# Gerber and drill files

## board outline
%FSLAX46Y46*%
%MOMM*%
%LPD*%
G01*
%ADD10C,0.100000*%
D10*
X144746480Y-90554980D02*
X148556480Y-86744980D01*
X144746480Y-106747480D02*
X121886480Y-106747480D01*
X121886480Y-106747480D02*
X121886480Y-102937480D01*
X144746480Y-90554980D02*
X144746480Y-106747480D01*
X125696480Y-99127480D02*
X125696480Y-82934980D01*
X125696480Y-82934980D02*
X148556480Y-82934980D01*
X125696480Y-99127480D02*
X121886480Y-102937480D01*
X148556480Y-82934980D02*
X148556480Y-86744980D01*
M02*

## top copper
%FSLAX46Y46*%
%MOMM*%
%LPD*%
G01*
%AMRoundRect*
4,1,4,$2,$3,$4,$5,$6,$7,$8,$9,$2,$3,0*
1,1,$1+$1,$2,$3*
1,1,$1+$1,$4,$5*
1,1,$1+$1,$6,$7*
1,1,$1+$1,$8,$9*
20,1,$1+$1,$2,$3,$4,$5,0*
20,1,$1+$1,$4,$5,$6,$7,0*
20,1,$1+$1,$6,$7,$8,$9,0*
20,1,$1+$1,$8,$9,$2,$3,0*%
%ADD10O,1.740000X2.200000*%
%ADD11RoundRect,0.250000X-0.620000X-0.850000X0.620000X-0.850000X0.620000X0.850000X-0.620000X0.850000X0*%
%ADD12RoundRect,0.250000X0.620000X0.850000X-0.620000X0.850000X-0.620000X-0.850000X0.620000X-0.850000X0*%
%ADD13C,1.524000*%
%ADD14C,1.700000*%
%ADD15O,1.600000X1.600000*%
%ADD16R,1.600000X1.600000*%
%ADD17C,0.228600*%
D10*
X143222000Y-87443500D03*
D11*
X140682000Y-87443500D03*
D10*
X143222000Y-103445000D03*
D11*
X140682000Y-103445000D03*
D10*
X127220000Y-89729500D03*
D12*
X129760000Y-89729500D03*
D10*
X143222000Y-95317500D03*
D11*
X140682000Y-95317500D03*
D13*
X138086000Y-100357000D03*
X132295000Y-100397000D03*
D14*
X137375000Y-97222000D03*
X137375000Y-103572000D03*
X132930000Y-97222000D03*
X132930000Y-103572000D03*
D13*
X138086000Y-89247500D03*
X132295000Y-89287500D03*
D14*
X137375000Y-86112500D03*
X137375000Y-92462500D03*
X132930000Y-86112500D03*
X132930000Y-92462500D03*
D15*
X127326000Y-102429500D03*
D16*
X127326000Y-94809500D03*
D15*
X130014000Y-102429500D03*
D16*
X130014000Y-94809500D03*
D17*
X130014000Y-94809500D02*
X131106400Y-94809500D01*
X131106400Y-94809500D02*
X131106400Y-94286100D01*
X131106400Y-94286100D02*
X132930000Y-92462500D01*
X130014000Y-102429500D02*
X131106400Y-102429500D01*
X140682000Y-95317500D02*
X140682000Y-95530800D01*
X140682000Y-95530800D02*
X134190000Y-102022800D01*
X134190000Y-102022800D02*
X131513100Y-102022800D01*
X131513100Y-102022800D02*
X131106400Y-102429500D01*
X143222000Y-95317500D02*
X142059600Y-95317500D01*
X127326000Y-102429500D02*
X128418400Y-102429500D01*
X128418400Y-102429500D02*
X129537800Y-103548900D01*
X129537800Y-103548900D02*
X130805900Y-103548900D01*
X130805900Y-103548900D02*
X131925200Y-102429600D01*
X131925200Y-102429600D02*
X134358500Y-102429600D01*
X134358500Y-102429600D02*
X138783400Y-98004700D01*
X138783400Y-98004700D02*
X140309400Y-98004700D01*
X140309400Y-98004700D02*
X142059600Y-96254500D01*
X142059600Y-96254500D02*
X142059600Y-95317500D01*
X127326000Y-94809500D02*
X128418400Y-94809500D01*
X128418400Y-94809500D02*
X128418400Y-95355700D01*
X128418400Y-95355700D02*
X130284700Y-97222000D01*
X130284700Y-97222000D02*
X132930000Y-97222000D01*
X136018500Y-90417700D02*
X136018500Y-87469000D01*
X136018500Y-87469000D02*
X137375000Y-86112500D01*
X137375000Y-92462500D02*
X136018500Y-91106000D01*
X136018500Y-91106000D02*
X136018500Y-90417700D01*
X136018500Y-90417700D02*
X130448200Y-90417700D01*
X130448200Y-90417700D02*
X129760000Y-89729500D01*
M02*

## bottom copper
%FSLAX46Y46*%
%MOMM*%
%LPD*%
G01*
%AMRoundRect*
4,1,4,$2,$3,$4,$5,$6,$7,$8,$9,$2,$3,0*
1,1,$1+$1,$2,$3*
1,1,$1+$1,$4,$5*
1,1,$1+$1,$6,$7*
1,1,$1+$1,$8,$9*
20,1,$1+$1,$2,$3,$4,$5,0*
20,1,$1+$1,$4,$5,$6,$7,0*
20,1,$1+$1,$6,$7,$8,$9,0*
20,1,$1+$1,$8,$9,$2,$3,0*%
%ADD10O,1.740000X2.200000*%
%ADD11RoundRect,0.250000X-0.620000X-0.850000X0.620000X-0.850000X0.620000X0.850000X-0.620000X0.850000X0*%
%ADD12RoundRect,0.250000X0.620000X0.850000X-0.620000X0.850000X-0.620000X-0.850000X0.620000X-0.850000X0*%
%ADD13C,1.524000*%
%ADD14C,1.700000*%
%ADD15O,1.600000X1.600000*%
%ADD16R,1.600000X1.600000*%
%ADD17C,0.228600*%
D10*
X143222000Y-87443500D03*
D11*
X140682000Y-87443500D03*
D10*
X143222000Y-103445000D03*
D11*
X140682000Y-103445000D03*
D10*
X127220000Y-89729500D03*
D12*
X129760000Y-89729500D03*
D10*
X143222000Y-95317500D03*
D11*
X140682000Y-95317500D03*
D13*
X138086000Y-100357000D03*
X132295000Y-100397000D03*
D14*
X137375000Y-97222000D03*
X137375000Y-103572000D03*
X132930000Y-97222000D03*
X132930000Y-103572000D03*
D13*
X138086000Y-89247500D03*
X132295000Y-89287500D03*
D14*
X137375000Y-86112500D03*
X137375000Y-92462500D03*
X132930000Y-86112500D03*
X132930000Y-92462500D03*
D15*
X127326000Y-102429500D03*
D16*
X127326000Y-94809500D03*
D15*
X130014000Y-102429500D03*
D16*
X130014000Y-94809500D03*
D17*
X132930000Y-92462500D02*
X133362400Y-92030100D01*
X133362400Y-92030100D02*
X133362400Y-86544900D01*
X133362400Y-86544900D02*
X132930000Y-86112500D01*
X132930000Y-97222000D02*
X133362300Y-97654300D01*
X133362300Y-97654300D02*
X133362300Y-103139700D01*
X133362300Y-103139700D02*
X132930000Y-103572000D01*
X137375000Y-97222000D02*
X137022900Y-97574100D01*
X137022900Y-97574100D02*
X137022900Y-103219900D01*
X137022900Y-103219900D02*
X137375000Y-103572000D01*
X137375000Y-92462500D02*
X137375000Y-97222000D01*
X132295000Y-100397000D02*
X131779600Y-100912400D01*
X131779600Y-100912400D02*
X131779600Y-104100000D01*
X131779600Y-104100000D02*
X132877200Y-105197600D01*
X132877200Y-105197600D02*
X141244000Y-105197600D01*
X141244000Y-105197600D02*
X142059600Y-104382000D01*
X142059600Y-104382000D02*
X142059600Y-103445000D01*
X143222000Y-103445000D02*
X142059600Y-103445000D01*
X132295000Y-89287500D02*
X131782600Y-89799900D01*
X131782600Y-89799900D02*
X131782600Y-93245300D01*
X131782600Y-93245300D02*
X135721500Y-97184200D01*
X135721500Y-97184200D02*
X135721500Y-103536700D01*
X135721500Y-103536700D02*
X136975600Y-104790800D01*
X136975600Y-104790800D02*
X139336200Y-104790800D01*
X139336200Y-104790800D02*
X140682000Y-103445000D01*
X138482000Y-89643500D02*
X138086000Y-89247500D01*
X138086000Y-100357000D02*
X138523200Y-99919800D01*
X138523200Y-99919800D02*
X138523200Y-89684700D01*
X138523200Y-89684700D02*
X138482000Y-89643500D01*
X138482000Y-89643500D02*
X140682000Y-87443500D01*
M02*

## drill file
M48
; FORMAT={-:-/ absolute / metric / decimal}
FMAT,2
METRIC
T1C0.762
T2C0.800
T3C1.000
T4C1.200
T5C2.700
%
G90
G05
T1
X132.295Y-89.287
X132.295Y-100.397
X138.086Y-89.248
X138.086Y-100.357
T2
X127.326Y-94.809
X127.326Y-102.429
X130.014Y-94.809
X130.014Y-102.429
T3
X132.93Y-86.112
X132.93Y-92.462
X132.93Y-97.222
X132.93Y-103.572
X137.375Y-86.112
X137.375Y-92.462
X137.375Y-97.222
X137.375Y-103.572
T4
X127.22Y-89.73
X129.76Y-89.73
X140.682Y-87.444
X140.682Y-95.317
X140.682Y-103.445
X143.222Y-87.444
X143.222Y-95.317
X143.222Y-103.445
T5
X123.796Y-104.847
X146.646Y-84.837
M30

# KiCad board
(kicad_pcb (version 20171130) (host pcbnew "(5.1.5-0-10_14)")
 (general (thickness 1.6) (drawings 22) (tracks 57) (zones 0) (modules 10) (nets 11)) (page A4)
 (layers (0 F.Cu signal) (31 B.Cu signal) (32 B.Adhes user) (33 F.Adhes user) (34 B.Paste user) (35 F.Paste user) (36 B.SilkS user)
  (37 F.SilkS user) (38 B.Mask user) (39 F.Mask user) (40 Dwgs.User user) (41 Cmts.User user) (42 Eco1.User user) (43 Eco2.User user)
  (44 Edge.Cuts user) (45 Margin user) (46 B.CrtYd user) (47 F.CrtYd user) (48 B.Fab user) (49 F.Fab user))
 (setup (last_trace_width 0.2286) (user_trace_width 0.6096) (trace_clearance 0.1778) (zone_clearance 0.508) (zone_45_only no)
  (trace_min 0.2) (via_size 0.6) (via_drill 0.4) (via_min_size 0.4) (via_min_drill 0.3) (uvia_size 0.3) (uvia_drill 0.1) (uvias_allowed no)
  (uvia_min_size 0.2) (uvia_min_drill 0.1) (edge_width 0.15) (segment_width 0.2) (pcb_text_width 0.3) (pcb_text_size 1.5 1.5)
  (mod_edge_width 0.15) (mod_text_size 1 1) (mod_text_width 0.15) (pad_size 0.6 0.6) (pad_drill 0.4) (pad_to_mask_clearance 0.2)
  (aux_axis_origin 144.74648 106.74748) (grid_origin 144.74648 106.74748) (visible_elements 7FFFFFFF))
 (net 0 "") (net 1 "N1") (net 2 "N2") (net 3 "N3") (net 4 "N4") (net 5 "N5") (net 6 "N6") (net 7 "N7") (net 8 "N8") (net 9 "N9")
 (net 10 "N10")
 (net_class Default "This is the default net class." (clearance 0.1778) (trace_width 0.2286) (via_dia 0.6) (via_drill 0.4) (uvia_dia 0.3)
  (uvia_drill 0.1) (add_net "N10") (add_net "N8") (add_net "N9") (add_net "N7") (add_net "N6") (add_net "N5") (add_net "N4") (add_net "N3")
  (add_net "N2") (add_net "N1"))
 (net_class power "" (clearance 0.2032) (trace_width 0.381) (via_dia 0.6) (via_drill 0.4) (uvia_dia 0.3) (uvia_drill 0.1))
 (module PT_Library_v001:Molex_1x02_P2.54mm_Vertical (layer B.Cu) (at 140.682 87.4435)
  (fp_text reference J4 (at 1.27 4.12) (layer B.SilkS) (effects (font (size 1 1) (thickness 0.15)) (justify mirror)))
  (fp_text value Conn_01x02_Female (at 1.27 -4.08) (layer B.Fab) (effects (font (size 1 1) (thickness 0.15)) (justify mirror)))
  (pad 2 thru_hole oval (at 2.54 0) (size 1.74 2.2) (drill 1.2) (layers *.Cu *.Mask) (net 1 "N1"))
  (pad 1 thru_hole roundrect (at 0 0) (size 1.74 2.2) (drill 1.2) (layers *.Cu *.Mask) (roundrect_rratio 0.143678) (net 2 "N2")))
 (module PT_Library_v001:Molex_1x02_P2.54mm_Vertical (layer B.Cu) (at 140.682 103.445)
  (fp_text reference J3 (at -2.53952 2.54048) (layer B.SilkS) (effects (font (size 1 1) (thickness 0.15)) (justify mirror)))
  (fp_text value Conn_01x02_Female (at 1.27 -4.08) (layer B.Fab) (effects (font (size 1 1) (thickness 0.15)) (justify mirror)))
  (pad 2 thru_hole oval (at 2.54 0) (size 1.74 2.2) (drill 1.2) (layers *.Cu *.Mask) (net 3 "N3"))
  (pad 1 thru_hole roundrect (at 0 0) (size 1.74 2.2) (drill 1.2) (layers *.Cu *.Mask) (roundrect_rratio 0.143678) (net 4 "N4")))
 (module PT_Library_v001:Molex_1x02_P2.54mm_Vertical (layer B.Cu) (at 129.76 89.7295 180)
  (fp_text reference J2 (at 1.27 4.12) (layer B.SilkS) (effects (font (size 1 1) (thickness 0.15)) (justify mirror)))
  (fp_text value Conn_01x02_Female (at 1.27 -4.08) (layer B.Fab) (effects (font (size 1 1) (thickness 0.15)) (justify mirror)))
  (pad 2 thru_hole oval (at 2.54 0 180) (size 1.74 2.2) (drill 1.2) (layers *.Cu *.Mask) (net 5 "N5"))
  (pad 1 thru_hole roundrect (at 0 0 180) (size 1.74 2.2) (drill 1.2) (layers *.Cu *.Mask) (roundrect_rratio 0.143678) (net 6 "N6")))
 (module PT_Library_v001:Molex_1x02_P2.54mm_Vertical (layer B.Cu) (at 140.682 95.3175)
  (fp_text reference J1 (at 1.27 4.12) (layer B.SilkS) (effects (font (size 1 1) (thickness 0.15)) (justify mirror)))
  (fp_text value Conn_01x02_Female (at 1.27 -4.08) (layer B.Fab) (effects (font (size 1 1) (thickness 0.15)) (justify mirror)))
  (pad 2 thru_hole oval (at 2.54 0) (size 1.74 2.2) (drill 1.2) (layers *.Cu *.Mask) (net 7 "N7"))
  (pad 1 thru_hole roundrect (at 0 0) (size 1.74 2.2) (drill 1.2) (layers *.Cu *.Mask) (roundrect_rratio 0.143678) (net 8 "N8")))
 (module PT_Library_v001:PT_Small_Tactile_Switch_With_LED (layer F.Cu) (at 135.216 100.397 90)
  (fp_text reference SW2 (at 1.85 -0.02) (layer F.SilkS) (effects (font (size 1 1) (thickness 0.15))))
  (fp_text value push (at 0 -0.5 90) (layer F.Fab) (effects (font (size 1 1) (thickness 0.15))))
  (pad 6 thru_hole circle (at 0.04 2.87 90) (size 1.524 1.524) (drill 0.762) (layers *.Cu *.Mask) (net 2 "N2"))
  (pad 5 thru_hole circle (at 0 -2.921 90) (size 1.524 1.524) (drill 0.762) (layers *.Cu *.Mask) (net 3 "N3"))
  (pad 4 thru_hole circle (at 3.175 2.159 90) (size 1.7 1.7) (drill 1) (layers *.Cu *.Mask) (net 6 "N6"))
  (pad 3 thru_hole circle (at -3.175 2.159 90) (size 1.7 1.7) (drill 1) (layers *.Cu *.Mask) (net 6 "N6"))
  (pad 2 thru_hole circle (at 3.175 -2.286 90) (size 1.7 1.7) (drill 1) (layers *.Cu *.Mask) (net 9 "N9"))
  (pad 1 thru_hole circle (at -3.175 -2.286 90) (size 1.7 1.7) (drill 1) (layers *.Cu *.Mask) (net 9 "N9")))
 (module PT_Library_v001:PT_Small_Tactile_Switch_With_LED (layer F.Cu) (at 135.216 89.2875 90)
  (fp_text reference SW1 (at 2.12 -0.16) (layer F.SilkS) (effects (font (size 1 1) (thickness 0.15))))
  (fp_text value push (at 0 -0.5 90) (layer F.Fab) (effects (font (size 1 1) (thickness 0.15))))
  (pad 6 thru_hole circle (at 0.04 2.87 90) (size 1.524 1.524) (drill 0.762) (layers *.Cu *.Mask) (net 2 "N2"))
  (pad 5 thru_hole circle (at 0 -2.921 90) (size 1.524 1.524) (drill 0.762) (layers *.Cu *.Mask) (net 4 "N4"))
  (pad 4 thru_hole circle (at 3.175 2.159 90) (size 1.7 1.7) (drill 1) (layers *.Cu *.Mask) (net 6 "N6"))
  (pad 3 thru_hole circle (at -3.175 2.159 90) (size 1.7 1.7) (drill 1) (layers *.Cu *.Mask) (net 6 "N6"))
  (pad 2 thru_hole circle (at 3.175 -2.286 90) (size 1.7 1.7) (drill 1) (layers *.Cu *.Mask) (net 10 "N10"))
  (pad 1 thru_hole circle (at -3.175 -2.286 90) (size 1.7 1.7) (drill 1) (layers *.Cu *.Mask) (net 10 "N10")))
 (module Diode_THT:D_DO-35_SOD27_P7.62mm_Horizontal (layer F.Cu) (at 127.326 94.8095 270)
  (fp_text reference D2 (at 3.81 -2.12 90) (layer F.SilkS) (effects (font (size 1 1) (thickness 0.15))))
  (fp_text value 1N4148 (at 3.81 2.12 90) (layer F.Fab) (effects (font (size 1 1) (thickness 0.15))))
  (pad 2 thru_hole oval (at 7.62 0 270) (size 1.6 1.6) (drill 0.8) (layers *.Cu *.Mask) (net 7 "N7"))
  (pad 1 thru_hole rect (at 0 0 270) (size 1.6 1.6) (drill 0.8) (layers *.Cu *.Mask) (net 9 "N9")))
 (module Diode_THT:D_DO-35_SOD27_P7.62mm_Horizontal (layer F.Cu) (at 130.014 94.8095 270)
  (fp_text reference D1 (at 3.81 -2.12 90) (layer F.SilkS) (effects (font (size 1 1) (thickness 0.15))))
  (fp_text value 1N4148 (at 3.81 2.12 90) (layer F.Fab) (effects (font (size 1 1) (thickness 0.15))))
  (pad 2 thru_hole oval (at 7.62 0 270) (size 1.6 1.6) (drill 0.8) (layers *.Cu *.Mask) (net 8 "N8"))
  (pad 1 thru_hole rect (at 0 0 270) (size 1.6 1.6) (drill 0.8) (layers *.Cu *.Mask) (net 10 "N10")))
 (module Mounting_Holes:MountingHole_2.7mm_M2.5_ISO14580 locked (layer F.Cu) (at 146.646 84.8375 180)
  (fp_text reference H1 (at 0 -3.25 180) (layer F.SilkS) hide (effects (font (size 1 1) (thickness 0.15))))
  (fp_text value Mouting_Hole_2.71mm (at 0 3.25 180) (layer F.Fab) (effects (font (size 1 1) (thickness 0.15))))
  (pad 1 np_thru_hole circle (at 0 0 180) (size 2.7 2.7) (drill 2.7) (layers *.Cu *.Mask)))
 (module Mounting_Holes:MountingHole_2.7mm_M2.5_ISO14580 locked (layer F.Cu) (at 123.796 104.847 180)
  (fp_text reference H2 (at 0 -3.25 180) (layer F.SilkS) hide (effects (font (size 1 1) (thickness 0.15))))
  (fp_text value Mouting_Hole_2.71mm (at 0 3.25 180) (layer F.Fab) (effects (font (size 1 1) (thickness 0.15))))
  (pad 1 np_thru_hole circle (at 0 0 180) (size 2.7 2.7) (drill 2.7) (layers *.Cu *.Mask)))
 (gr_line (start 144.74648 90.55498) (end 148.55648 86.74498) (layer Edge.Cuts) (width 0.1))
 (gr_line (start 144.74648 106.74748) (end 121.88648 106.74748) (layer Edge.Cuts) (width 0.1))
 (gr_line (start 121.88648 106.74748) (end 121.88648 102.93748) (layer Edge.Cuts) (width 0.1))
 (gr_line (start 144.74648 90.55498) (end 144.74648 106.74748) (layer Edge.Cuts) (width 0.1))
 (gr_line (start 125.69648 99.12748) (end 125.69648 82.93498) (layer Edge.Cuts) (width 0.1))
 (gr_line (start 125.69648 82.93498) (end 148.55648 82.93498) (layer Edge.Cuts) (width 0.1))
 (gr_line (start 125.69648 99.12748) (end 121.88648 102.93748) (layer Edge.Cuts) (width 0.1))
 (gr_line (start 148.55648 82.93498) (end 148.55648 86.74498) (layer Edge.Cuts) (width 0.1))
 (segment (start 130.014 94.8095) (end 131.1064 94.8095) (width 0.2286) (layer F.Cu) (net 10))
 (segment (start 131.1064 94.8095) (end 131.1064 94.2861) (width 0.2286) (layer F.Cu) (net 10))
 (segment (start 131.1064 94.2861) (end 132.93 92.4625) (width 0.2286) (layer F.Cu) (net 10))
 (segment (start 132.93 92.4625) (end 133.3624 92.0301) (width 0.2286) (layer B.Cu) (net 10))
 (segment (start 133.3624 92.0301) (end 133.3624 86.5449) (width 0.2286) (layer B.Cu) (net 10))
 (segment (start 133.3624 86.5449) (end 132.93 86.1125) (width 0.2286) (layer B.Cu) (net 10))
 (segment (start 130.014 102.4295) (end 131.1064 102.4295) (width 0.2286) (layer F.Cu) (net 8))
 (segment (start 140.682 95.3175) (end 140.682 95.5308) (width 0.2286) (layer F.Cu) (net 8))
 (segment (start 140.682 95.5308) (end 134.19 102.0228) (width 0.2286) (layer F.Cu) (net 8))
 (segment (start 134.19 102.0228) (end 131.5131 102.0228) (width 0.2286) (layer F.Cu) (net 8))
 (segment (start 131.5131 102.0228) (end 131.1064 102.4295) (width 0.2286) (layer F.Cu) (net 8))
 (segment (start 143.222 95.3175) (end 142.0596 95.3175) (width 0.2286) (layer F.Cu) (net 7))
 (segment (start 127.326 102.4295) (end 128.4184 102.4295) (width 0.2286) (layer F.Cu) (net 7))
 (segment (start 128.4184 102.4295) (end 129.5378 103.5489) (width 0.2286) (layer F.Cu) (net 7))
 (segment (start 129.5378 103.5489) (end 130.8059 103.5489) (width 0.2286) (layer F.Cu) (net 7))
 (segment (start 130.8059 103.5489) (end 131.9252 102.4296) (width 0.2286) (layer F.Cu) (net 7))
 (segment (start 131.9252 102.4296) (end 134.3585 102.4296) (width 0.2286) (layer F.Cu) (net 7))
 (segment (start 134.3585 102.4296) (end 138.7834 98.0047) (width 0.2286) (layer F.Cu) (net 7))
 (segment (start 138.7834 98.0047) (end 140.3094 98.0047) (width 0.2286) (layer F.Cu) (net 7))
 (segment (start 140.3094 98.0047) (end 142.0596 96.2545) (width 0.2286) (layer F.Cu) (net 7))
 (segment (start 142.0596 96.2545) (end 142.0596 95.3175) (width 0.2286) (layer F.Cu) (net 7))
 (segment (start 132.93 97.222) (end 133.3623 97.6543) (width 0.2286) (layer B.Cu) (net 9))
 (segment (start 133.3623 97.6543) (end 133.3623 103.1397) (width 0.2286) (layer B.Cu) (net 9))
 (segment (start 133.3623 103.1397) (end 132.93 103.572) (width 0.2286) (layer B.Cu) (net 9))
 (segment (start 127.326 94.8095) (end 128.4184 94.8095) (width 0.2286) (layer F.Cu) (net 9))
 (segment (start 128.4184 94.8095) (end 128.4184 95.3557) (width 0.2286) (layer F.Cu) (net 9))
 (segment (start 128.4184 95.3557) (end 130.2847 97.222) (width 0.2286) (layer F.Cu) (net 9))
 (segment (start 130.2847 97.222) (end 132.93 97.222) (width 0.2286) (layer F.Cu) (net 9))
 (segment (start 136.0185 90.4177) (end 136.0185 87.469) (width 0.2286) (layer F.Cu) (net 6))
 (segment (start 136.0185 87.469) (end 137.375 86.1125) (width 0.2286) (layer F.Cu) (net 6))
 (segment (start 137.375 92.4625) (end 136.0185 91.106) (width 0.2286) (layer F.Cu) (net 6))
 (segment (start 136.0185 91.106) (end 136.0185 90.4177) (width 0.2286) (layer F.Cu) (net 6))
 (segment (start 136.0185 90.4177) (end 130.4482 90.4177) (width 0.2286) (layer F.Cu) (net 6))
 (segment (start 130.4482 90.4177) (end 129.76 89.7295) (width 0.2286) (layer F.Cu) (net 6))
 (segment (start 137.375 97.222) (end 137.0229 97.5741) (width 0.2286) (layer B.Cu) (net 6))
 (segment (start 137.0229 97.5741) (end 137.0229 103.2199) (width 0.2286) (layer B.Cu) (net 6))
 (segment (start 137.0229 103.2199) (end 137.375 103.572) (width 0.2286) (layer B.Cu) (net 6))
 (segment (start 137.375 92.4625) (end 137.375 97.222) (width 0.2286) (layer B.Cu) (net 6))
 (segment (start 132.295 100.397) (end 131.7796 100.9124) (width 0.2286) (layer B.Cu) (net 3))
 (segment (start 131.7796 100.9124) (end 131.7796 104.1) (width 0.2286) (layer B.Cu) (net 3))
 (segment (start 131.7796 104.1) (end 132.8772 105.1976) (width 0.2286) (layer B.Cu) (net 3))
 (segment (start 132.8772 105.1976) (end 141.244 105.1976) (width 0.2286) (layer B.Cu) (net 3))
 (segment (start 141.244 105.1976) (end 142.0596 104.382) (width 0.2286) (layer B.Cu) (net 3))
 (segment (start 142.0596 104.382) (end 142.0596 103.445) (width 0.2286) (layer B.Cu) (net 3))
 (segment (start 143.222 103.445) (end 142.0596 103.445) (width 0.2286) (layer B.Cu) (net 3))
 (segment (start 132.295 89.2875) (end 131.7826 89.7999) (width 0.2286) (layer B.Cu) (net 4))
 (segment (start 131.7826 89.7999) (end 131.7826 93.2453) (width 0.2286) (layer B.Cu) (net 4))
 (segment (start 131.7826 93.2453) (end 135.7215 97.1842) (width 0.2286) (layer B.Cu) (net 4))
 (segment (start 135.7215 97.1842) (end 135.7215 103.5367) (width 0.2286) (layer B.Cu) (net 4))
 (segment (start 135.7215 103.5367) (end 136.9756 104.7908) (width 0.2286) (layer B.Cu) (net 4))
 (segment (start 136.9756 104.7908) (end 139.3362 104.7908) (width 0.2286) (layer B.Cu) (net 4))
 (segment (start 139.3362 104.7908) (end 140.682 103.445) (width 0.2286) (layer B.Cu) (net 4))
 (segment (start 138.482 89.6435) (end 138.086 89.2475) (width 0.2286) (layer B.Cu) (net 2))
 (segment (start 138.086 100.357) (end 138.5232 99.9198) (width 0.2286) (layer B.Cu) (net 2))
 (segment (start 138.5232 99.9198) (end 138.5232 89.6847) (width 0.2286) (layer B.Cu) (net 2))
 (segment (start 138.5232 89.6847) (end 138.482 89.6435) (width 0.2286) (layer B.Cu) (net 2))
 (segment (start 138.482 89.6435) (end 140.682 87.4435) (width 0.2286) (layer B.Cu) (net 2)))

